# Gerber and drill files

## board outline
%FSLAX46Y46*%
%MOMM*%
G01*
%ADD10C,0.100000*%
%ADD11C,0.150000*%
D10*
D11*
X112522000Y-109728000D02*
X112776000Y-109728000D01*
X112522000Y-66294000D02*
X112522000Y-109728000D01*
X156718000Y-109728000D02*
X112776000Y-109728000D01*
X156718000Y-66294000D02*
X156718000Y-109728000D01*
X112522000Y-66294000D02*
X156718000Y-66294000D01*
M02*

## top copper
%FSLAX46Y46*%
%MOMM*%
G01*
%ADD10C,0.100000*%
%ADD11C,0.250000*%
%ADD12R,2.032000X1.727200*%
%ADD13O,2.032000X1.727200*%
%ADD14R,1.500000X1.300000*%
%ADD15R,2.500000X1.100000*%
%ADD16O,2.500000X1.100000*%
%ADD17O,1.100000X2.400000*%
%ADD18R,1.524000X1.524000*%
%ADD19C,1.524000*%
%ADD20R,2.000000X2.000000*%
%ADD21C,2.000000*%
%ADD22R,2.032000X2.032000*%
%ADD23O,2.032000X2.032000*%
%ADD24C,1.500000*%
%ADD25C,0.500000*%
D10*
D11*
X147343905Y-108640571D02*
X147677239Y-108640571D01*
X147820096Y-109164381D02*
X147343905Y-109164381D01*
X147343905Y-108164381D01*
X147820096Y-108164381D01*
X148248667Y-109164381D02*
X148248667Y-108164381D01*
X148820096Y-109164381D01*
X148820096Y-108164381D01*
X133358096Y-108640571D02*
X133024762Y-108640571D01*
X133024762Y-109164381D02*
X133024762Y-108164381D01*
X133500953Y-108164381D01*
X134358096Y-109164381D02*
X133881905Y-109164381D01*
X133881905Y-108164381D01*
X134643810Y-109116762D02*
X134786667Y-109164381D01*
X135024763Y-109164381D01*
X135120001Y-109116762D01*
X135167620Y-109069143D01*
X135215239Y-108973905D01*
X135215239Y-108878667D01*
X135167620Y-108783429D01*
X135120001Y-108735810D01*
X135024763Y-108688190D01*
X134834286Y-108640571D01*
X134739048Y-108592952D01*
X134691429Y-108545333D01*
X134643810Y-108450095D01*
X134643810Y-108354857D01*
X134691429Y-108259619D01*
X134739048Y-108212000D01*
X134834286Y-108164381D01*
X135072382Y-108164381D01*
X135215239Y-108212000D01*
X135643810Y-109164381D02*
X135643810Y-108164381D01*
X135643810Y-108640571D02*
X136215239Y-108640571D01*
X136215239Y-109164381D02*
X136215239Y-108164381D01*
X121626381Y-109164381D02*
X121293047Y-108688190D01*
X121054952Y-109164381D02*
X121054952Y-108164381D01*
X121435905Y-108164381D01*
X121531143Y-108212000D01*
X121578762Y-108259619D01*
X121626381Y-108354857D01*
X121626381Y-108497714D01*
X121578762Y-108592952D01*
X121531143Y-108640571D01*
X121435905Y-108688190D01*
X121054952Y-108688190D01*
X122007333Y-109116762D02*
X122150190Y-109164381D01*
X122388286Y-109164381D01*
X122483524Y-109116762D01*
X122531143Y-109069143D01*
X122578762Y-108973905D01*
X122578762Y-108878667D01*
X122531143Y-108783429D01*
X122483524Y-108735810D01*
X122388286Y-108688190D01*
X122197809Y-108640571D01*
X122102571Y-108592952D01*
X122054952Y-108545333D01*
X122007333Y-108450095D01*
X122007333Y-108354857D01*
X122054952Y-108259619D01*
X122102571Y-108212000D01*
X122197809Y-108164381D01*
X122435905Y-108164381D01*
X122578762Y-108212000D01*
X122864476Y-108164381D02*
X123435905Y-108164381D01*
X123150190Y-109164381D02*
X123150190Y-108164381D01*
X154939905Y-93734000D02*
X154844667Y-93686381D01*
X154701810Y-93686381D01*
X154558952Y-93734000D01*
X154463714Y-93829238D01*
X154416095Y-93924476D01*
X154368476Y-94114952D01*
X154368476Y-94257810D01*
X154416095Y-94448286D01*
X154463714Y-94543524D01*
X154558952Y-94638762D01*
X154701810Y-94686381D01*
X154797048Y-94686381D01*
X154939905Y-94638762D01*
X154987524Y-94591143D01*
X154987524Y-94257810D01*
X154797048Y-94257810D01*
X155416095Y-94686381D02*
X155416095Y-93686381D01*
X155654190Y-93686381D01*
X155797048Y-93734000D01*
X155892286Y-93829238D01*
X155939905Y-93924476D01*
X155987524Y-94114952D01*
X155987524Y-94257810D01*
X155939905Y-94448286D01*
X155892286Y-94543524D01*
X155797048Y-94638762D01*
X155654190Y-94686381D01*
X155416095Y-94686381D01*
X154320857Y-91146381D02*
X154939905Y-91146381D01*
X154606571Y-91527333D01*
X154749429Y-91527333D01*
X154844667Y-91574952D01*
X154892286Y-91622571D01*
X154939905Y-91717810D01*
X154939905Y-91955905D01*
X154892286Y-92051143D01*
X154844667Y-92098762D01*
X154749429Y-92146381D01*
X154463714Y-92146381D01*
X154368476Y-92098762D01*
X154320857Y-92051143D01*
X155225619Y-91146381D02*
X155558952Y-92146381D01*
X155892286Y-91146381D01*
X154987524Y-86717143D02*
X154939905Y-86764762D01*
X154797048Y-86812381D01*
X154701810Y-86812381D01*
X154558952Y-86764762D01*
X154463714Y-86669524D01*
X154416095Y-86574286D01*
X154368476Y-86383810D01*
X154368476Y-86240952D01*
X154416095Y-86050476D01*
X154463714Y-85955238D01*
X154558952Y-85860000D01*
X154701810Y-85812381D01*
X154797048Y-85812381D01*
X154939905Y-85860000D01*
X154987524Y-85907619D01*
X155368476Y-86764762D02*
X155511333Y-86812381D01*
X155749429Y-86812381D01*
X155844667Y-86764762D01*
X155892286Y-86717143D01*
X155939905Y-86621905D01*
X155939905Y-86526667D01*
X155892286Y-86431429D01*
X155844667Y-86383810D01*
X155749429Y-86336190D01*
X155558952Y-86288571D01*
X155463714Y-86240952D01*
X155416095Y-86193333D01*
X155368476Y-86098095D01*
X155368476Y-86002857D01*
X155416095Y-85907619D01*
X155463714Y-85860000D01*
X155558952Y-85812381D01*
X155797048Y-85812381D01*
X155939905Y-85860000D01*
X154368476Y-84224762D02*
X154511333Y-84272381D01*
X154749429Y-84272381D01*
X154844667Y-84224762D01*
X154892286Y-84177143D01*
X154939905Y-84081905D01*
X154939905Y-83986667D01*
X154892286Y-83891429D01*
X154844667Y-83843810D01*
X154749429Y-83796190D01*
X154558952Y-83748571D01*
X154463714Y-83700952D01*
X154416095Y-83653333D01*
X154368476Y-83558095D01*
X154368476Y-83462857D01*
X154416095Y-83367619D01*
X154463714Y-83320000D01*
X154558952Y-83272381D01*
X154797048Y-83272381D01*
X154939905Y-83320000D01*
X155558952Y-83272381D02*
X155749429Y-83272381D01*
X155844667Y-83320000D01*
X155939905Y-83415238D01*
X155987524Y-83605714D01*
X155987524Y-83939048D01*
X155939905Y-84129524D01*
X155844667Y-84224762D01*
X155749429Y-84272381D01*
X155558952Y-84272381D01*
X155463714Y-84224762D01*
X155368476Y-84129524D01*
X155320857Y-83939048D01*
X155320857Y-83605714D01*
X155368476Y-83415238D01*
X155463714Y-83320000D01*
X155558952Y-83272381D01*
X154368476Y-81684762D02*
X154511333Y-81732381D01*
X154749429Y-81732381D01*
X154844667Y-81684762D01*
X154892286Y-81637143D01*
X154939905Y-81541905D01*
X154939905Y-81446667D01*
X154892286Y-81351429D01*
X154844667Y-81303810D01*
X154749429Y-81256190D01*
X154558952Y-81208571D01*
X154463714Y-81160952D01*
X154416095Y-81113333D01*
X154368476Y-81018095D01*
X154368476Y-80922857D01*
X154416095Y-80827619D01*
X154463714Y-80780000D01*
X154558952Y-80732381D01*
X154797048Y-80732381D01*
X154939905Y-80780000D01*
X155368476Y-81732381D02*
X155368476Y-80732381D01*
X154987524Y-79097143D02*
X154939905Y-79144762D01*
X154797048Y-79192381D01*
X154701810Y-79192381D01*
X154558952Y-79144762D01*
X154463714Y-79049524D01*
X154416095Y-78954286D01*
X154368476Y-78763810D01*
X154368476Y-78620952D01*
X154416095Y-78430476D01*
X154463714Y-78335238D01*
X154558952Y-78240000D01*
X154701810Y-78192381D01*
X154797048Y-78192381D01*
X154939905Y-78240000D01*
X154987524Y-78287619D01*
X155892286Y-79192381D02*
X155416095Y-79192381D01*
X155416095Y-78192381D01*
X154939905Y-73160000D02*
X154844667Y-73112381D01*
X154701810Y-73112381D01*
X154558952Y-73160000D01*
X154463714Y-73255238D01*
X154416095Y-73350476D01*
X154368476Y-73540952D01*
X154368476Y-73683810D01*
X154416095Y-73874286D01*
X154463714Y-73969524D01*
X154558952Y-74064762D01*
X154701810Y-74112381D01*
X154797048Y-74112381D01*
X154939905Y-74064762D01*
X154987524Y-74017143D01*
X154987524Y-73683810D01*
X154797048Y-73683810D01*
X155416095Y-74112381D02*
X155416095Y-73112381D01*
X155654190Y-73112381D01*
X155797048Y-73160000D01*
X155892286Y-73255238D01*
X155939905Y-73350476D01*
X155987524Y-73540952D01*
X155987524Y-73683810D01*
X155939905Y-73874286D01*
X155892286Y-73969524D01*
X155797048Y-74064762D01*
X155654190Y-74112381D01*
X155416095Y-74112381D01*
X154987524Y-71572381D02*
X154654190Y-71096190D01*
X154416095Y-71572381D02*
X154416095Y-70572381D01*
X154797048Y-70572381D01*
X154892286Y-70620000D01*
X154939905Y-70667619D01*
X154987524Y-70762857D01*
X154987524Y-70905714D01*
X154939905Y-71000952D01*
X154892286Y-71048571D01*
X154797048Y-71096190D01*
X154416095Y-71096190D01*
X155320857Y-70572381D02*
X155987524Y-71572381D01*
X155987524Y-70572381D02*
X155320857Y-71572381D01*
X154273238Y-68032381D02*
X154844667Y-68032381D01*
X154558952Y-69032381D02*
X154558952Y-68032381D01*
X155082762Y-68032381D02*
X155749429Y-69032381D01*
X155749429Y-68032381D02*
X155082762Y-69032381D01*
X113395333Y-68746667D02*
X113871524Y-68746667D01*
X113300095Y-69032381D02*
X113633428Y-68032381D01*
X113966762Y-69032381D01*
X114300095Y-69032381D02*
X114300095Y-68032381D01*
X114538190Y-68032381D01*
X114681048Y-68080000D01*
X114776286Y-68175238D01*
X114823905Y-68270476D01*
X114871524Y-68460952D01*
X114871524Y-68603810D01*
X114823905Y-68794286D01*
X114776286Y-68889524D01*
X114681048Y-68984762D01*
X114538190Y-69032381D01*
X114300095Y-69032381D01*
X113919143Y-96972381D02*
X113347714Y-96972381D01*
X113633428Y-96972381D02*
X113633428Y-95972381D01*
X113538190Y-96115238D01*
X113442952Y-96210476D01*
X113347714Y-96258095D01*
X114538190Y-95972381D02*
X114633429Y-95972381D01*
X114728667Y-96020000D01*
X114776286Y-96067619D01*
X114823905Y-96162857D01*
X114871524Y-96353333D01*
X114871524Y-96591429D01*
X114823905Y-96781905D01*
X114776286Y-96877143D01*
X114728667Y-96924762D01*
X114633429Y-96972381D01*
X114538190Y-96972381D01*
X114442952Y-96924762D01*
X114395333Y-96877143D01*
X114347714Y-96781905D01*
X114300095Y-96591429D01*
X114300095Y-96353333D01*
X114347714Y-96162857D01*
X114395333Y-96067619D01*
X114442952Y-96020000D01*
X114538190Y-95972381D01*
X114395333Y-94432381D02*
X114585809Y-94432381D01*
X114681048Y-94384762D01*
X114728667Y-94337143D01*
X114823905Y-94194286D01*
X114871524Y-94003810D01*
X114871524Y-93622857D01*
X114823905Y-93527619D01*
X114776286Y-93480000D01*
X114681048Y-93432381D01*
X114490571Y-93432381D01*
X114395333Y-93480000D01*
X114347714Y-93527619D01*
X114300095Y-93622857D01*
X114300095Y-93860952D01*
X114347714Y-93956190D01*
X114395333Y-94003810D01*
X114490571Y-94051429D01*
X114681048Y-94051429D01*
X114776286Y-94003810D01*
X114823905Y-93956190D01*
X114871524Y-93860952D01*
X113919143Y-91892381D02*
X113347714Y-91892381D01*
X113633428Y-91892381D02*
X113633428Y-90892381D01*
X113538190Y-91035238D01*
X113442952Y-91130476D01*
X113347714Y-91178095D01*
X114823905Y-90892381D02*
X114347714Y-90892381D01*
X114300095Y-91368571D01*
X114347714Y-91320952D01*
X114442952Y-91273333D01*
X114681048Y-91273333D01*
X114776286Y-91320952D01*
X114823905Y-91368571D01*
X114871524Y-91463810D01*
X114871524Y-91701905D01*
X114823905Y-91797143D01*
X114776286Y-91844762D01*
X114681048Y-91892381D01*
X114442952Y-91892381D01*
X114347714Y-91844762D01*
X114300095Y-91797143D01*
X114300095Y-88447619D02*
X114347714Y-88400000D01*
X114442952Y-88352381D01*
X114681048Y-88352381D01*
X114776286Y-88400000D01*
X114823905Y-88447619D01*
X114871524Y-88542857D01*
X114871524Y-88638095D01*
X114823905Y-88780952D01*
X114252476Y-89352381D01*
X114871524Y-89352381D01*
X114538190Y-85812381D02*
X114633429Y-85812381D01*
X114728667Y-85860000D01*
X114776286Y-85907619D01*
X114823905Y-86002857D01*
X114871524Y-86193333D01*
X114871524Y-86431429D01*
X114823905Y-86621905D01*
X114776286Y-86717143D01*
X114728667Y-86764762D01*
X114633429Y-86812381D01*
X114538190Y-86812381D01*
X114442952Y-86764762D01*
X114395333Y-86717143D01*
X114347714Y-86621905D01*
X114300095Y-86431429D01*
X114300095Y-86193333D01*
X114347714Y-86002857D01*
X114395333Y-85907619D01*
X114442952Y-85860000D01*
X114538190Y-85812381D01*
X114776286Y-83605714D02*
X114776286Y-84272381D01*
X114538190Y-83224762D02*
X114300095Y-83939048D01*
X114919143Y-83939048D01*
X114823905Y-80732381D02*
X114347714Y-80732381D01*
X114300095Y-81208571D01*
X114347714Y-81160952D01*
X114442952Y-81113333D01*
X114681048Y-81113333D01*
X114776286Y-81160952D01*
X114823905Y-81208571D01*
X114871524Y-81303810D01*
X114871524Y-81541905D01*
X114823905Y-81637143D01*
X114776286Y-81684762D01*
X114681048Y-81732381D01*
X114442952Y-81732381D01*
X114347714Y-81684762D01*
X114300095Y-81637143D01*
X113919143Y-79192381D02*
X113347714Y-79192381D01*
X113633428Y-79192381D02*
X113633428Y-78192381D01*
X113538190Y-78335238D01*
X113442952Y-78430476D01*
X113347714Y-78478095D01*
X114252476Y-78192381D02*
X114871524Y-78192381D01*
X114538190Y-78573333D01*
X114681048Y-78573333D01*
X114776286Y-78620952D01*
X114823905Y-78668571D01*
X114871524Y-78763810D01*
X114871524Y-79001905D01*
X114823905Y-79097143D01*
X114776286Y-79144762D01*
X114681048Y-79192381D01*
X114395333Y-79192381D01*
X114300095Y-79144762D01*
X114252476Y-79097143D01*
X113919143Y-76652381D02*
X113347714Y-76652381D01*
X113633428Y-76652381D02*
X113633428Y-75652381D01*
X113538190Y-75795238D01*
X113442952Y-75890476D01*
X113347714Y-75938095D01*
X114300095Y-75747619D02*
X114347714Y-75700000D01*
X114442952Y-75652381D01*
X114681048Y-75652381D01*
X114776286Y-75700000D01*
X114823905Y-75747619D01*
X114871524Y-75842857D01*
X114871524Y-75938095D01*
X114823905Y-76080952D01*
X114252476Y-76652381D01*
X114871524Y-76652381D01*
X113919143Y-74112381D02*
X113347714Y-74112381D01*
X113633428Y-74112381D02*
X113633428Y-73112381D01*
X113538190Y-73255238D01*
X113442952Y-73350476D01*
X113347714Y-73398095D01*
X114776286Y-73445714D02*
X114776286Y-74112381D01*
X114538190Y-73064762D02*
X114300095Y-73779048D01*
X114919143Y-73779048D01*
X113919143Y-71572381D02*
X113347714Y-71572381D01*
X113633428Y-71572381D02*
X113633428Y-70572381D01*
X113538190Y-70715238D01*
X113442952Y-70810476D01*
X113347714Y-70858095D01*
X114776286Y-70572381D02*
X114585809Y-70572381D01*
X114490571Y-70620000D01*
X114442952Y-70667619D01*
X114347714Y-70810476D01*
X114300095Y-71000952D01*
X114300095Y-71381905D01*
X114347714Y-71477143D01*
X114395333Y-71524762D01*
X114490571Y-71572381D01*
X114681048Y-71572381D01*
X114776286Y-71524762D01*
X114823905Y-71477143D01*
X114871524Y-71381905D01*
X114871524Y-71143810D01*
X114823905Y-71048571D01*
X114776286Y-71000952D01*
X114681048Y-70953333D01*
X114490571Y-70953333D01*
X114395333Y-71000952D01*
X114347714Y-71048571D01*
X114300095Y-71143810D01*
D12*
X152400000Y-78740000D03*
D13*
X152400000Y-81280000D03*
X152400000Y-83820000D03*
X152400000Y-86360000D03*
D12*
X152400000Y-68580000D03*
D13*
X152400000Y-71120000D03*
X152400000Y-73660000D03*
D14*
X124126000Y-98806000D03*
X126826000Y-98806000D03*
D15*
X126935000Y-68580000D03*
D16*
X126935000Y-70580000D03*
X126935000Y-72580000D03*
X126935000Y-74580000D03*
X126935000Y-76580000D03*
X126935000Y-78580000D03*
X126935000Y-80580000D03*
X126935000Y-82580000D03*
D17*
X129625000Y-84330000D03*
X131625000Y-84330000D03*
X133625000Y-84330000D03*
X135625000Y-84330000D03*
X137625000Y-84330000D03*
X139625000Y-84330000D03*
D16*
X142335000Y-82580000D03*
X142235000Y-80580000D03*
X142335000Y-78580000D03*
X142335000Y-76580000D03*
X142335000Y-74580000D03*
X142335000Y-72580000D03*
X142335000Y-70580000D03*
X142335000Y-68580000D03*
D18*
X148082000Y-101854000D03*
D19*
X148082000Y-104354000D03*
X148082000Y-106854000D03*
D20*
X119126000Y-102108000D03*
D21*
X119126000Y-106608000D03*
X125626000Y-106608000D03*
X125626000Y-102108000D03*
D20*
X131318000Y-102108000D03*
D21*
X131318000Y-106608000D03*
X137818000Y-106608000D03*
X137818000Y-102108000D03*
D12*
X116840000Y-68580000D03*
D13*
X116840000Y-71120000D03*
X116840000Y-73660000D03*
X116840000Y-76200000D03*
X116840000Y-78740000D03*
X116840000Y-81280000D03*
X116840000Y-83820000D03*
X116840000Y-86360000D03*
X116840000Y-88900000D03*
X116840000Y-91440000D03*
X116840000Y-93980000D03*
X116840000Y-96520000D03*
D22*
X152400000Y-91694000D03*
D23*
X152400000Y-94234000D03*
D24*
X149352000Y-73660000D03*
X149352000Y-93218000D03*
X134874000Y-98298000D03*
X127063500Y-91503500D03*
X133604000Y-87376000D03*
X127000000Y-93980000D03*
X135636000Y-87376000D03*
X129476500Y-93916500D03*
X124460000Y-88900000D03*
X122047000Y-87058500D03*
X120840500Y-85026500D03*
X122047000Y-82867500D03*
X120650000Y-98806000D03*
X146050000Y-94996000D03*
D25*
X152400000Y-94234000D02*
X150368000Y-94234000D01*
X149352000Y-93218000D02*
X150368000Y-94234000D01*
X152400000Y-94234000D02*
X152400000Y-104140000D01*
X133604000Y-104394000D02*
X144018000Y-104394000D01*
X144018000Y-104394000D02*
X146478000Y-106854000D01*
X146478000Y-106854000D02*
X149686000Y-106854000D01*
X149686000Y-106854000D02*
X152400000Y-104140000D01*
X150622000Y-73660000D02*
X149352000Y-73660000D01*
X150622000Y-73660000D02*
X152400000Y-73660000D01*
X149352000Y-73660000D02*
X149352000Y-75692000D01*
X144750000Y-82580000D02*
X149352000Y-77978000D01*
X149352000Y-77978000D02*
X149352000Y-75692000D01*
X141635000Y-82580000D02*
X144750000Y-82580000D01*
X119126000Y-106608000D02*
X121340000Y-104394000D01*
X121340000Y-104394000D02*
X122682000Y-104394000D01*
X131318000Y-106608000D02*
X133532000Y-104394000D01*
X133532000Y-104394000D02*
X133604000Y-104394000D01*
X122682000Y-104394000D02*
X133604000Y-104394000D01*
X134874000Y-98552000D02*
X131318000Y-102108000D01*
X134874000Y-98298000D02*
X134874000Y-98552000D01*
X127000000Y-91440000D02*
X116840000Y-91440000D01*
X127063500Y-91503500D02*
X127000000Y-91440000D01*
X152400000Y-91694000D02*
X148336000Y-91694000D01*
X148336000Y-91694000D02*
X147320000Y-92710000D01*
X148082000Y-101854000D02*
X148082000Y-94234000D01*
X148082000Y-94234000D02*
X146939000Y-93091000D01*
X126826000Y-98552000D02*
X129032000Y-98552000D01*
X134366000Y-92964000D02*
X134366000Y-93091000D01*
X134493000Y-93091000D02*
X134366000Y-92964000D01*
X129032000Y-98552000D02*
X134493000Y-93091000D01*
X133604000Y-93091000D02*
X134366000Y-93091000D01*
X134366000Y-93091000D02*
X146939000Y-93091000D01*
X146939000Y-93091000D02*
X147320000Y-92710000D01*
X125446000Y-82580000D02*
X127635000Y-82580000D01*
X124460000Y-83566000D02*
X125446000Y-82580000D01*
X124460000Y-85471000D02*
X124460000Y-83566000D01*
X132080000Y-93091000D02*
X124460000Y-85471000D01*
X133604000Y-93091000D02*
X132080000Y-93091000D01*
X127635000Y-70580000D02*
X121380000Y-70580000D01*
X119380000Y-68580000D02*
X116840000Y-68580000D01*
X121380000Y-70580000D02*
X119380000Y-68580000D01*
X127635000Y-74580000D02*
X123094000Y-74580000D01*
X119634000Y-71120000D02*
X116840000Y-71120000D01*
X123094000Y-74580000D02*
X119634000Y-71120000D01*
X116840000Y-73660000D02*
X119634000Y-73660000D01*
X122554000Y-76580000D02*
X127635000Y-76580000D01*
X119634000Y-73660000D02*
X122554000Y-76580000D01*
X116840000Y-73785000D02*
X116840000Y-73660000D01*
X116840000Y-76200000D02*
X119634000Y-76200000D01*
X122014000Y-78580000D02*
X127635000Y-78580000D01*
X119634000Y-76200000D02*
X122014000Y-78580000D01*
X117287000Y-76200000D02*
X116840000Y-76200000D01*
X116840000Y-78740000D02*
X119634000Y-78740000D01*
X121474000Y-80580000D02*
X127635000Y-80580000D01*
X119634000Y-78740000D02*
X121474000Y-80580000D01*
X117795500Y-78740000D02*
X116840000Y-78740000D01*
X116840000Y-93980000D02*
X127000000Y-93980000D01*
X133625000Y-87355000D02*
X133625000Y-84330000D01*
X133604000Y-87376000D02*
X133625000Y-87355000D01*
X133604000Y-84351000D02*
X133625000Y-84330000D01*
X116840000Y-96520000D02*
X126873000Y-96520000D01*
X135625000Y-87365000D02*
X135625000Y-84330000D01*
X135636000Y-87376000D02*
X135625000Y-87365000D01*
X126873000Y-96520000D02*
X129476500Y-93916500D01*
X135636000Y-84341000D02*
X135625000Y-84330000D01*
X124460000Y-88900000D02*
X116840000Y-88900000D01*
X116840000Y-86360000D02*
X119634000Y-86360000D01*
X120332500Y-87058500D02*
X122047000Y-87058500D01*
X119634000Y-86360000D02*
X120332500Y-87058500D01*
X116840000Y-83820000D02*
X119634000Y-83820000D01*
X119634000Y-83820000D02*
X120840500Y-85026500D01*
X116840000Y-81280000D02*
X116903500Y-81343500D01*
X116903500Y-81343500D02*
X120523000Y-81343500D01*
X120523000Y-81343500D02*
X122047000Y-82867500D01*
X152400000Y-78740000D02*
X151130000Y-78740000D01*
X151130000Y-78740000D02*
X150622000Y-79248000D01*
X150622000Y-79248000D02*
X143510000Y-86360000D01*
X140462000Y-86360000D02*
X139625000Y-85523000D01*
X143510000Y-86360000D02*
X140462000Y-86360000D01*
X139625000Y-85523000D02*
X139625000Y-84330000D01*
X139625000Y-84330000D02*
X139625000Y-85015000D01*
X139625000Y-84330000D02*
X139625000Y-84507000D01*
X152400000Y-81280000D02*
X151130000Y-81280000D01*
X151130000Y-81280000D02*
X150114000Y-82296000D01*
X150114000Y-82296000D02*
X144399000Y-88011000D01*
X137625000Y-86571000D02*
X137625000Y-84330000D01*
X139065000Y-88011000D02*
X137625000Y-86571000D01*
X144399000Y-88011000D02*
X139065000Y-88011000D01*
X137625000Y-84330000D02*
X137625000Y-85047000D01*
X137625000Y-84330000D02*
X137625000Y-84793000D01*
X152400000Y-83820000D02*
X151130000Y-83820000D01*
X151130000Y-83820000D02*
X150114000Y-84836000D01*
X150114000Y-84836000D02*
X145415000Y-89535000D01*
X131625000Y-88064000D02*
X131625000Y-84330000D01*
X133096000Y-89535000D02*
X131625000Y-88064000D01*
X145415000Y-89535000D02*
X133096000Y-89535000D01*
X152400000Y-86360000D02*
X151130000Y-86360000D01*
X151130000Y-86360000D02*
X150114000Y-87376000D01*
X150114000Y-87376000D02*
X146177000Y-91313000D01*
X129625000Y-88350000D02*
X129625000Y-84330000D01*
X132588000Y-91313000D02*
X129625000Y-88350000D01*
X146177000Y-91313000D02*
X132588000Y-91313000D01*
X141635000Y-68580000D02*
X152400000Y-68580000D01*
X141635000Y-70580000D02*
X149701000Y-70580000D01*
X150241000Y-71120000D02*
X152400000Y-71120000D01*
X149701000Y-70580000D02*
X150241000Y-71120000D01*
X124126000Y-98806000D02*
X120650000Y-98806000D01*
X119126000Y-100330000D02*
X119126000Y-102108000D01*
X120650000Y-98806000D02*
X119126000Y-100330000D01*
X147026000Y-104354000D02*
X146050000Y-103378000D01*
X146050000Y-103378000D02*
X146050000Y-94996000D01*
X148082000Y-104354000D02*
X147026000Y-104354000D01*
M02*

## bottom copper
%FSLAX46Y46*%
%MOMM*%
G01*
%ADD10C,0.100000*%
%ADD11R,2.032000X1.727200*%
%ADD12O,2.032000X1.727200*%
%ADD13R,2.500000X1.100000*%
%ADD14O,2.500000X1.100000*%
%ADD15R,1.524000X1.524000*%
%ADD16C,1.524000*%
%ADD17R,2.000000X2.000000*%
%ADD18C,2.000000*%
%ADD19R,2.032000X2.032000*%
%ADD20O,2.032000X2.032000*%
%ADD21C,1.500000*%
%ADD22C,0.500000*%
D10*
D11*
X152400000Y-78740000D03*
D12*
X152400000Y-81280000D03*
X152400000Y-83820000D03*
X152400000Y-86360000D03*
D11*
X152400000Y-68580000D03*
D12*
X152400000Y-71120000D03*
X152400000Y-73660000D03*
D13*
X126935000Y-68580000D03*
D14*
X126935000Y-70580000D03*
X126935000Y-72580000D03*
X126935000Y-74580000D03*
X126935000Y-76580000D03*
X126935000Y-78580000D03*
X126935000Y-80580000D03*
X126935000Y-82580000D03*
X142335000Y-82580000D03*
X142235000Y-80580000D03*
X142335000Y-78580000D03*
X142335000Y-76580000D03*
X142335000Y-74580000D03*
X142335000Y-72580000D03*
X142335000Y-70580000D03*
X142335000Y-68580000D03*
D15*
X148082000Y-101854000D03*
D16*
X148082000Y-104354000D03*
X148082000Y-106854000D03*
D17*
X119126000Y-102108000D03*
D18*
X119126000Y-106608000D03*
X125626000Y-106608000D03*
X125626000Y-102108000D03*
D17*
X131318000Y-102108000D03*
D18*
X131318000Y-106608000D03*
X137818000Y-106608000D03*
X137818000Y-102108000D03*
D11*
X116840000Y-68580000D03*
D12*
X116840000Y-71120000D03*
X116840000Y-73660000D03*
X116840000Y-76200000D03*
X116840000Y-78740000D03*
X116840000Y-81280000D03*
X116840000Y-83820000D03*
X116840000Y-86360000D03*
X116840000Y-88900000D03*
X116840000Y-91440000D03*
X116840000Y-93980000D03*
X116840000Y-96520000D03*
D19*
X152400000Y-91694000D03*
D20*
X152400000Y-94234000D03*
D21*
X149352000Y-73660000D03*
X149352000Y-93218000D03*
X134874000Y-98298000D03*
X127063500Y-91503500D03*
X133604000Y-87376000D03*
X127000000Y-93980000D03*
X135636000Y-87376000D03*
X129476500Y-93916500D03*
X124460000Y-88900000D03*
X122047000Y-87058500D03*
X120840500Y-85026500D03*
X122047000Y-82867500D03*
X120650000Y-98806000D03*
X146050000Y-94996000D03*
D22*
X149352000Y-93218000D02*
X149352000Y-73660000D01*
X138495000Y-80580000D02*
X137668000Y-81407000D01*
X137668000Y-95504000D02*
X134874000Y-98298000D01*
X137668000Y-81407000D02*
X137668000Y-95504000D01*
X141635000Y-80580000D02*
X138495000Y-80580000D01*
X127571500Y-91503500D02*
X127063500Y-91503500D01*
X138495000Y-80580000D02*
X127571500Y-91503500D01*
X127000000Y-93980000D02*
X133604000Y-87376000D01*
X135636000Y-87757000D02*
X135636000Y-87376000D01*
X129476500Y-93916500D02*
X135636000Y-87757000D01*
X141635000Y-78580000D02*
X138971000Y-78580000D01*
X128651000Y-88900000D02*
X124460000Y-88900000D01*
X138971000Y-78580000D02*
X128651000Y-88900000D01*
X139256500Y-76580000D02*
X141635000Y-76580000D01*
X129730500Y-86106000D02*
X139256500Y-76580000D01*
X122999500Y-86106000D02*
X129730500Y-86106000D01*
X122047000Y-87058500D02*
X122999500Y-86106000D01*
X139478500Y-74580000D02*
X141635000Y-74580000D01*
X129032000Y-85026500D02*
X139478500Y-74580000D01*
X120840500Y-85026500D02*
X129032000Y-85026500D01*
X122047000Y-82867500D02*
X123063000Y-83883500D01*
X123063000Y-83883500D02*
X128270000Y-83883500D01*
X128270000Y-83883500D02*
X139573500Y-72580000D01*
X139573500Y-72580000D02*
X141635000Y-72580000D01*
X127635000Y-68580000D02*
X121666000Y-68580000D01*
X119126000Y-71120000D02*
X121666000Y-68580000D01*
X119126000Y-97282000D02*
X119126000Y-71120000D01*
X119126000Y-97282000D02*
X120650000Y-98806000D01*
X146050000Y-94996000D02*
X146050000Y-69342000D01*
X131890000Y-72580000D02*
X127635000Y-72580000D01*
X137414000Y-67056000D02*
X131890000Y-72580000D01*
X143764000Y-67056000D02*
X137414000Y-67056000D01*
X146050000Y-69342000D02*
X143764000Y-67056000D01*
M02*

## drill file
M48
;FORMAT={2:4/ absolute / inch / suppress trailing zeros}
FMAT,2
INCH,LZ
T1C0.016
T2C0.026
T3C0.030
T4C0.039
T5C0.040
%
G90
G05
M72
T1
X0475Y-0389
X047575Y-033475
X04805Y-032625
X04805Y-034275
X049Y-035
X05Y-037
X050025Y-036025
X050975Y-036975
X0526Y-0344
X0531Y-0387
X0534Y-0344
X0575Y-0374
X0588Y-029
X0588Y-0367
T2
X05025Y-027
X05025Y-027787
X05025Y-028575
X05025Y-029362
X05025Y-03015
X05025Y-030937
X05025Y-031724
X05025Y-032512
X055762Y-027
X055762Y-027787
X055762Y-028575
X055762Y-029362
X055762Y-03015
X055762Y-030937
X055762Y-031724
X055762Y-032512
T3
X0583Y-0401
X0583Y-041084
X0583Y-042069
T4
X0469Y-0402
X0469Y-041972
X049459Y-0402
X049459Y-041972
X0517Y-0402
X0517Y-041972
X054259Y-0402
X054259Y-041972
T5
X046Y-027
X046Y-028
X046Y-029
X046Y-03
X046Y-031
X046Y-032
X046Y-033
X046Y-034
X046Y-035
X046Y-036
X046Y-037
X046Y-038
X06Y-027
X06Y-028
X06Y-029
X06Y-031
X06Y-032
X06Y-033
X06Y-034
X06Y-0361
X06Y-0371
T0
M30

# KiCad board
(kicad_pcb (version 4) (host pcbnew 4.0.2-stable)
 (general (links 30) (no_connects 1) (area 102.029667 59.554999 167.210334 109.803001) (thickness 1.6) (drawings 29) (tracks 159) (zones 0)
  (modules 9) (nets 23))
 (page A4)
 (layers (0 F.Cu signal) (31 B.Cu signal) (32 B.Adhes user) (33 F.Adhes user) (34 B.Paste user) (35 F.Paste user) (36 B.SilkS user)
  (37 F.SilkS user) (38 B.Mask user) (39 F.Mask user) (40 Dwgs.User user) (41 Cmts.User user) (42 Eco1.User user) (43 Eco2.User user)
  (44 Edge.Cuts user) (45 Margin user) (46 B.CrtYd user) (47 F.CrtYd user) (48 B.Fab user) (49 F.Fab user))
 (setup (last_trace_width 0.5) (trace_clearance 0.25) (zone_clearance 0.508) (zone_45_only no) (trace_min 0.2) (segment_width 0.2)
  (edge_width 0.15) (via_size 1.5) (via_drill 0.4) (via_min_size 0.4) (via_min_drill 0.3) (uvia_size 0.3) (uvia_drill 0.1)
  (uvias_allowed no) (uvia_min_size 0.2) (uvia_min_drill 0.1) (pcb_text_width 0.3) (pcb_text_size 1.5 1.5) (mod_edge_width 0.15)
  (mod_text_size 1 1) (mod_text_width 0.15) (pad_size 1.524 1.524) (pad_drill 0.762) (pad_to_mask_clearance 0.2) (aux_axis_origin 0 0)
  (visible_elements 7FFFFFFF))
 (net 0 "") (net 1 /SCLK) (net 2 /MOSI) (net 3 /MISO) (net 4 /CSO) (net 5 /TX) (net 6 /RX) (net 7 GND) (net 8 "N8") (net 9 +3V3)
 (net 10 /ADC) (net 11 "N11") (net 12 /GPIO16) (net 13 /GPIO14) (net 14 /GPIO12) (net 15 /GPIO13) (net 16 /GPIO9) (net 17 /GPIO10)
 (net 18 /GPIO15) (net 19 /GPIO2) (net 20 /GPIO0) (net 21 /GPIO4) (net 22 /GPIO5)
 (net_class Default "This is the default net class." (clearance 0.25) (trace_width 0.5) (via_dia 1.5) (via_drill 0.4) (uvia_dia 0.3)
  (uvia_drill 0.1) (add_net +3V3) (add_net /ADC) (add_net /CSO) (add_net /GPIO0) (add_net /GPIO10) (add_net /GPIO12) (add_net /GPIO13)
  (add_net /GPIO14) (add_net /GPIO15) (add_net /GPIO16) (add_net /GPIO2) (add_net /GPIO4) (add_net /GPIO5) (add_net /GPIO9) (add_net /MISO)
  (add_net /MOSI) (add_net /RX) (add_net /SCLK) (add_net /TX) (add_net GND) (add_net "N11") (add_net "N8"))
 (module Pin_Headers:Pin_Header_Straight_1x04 (layer F.Cu) (at 152.4 78.74)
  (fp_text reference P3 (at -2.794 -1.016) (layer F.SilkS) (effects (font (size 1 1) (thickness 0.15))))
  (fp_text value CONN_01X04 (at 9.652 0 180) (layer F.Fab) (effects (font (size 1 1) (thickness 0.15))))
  (pad 1 thru_hole rect (at 0 0) (size 2.032 1.7272) (drill 1.016) (layers *.Cu *.Mask F.SilkS) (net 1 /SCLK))
  (pad 2 thru_hole oval (at 0 2.54) (size 2.032 1.7272) (drill 1.016) (layers *.Cu *.Mask F.SilkS) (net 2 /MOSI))
  (pad 3 thru_hole oval (at 0 5.08) (size 2.032 1.7272) (drill 1.016) (layers *.Cu *.Mask F.SilkS) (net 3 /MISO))
  (pad 4 thru_hole oval (at 0 7.62) (size 2.032 1.7272) (drill 1.016) (layers *.Cu *.Mask F.SilkS) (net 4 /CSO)))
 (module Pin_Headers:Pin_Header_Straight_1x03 (layer F.Cu) (at 152.4 68.58)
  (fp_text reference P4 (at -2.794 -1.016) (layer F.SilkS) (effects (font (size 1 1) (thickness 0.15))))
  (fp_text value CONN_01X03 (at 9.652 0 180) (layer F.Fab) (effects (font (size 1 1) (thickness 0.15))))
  (pad 1 thru_hole rect (at 0 0) (size 2.032 1.7272) (drill 1.016) (layers *.Cu *.Mask F.SilkS) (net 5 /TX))
  (pad 2 thru_hole oval (at 0 2.54) (size 2.032 1.7272) (drill 1.016) (layers *.Cu *.Mask F.SilkS) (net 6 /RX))
  (pad 3 thru_hole oval (at 0 5.08) (size 2.032 1.7272) (drill 1.016) (layers *.Cu *.Mask F.SilkS) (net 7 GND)))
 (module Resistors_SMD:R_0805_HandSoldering (layer F.Cu) (at 125.476 98.806)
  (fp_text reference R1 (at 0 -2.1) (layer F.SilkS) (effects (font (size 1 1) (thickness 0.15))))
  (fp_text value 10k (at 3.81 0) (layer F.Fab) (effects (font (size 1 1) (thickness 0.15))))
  (pad 1 smd rect (at -1.35 0) (size 1.5 1.3) (layers F.Cu F.Paste F.Mask) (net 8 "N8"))
  (pad 2 smd rect (at 1.35 0) (size 1.5 1.3) (layers F.Cu F.Paste F.Mask) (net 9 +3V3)))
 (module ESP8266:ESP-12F (layer F.Cu) (at 127.635 68.58)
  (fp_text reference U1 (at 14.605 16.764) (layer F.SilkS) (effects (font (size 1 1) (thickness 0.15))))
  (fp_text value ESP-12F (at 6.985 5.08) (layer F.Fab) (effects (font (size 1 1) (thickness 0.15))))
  (pad 1 thru_hole rect (at 0 0) (size 2.5 1.1) (drill 0.65 (offset -0.7 0)) (layers *.Cu *.Mask F.SilkS) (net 8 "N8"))
  (pad 2 thru_hole oval (at 0 2) (size 2.5 1.1) (drill 0.65 (offset -0.7 0)) (layers *.Cu *.Mask F.SilkS) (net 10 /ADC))
  (pad 3 thru_hole oval (at 0 4) (size 2.5 1.1) (drill 0.65 (offset -0.7 0)) (layers *.Cu *.Mask F.SilkS) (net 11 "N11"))
  (pad 4 thru_hole oval (at 0 6) (size 2.5 1.1) (drill 0.65 (offset -0.7 0)) (layers *.Cu *.Mask F.SilkS) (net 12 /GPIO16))
  (pad 5 thru_hole oval (at 0 8) (size 2.5 1.1) (drill 0.65 (offset -0.7 0)) (layers *.Cu *.Mask F.SilkS) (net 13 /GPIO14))
  (pad 6 thru_hole oval (at 0 10) (size 2.5 1.1) (drill 0.65 (offset -0.7 0)) (layers *.Cu *.Mask F.SilkS) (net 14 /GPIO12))
  (pad 7 thru_hole oval (at 0 12) (size 2.5 1.1) (drill 0.65 (offset -0.7 0)) (layers *.Cu *.Mask F.SilkS) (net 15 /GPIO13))
  (pad 8 thru_hole oval (at 0 14) (size 2.5 1.1) (drill 0.65 (offset -0.7 0)) (layers *.Cu *.Mask F.SilkS) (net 9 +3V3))
  (pad 9 smd oval (at 1.99 15.75 90) (size 2.4 1.1) (layers F.Cu F.Paste F.Mask) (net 4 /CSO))
  (pad 10 smd oval (at 3.99 15.75 90) (size 2.4 1.1) (layers F.Cu F.Paste F.Mask) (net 3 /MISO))
  (pad 11 smd oval (at 5.99 15.75 90) (size 2.4 1.1) (layers F.Cu F.Paste F.Mask) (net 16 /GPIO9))
  (pad 12 smd oval (at 7.99 15.75 90) (size 2.4 1.1) (layers F.Cu F.Paste F.Mask) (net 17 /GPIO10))
  (pad 13 smd oval (at 9.99 15.75 90) (size 2.4 1.1) (layers F.Cu F.Paste F.Mask) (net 2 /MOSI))
  (pad 14 smd oval (at 11.99 15.75 90) (size 2.4 1.1) (layers F.Cu F.Paste F.Mask) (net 1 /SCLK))
  (pad 15 thru_hole oval (at 14 14) (size 2.5 1.1) (drill 0.65 (offset 0.7 0)) (layers *.Cu *.Mask F.SilkS) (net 7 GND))
  (pad 16 thru_hole oval (at 14 12) (size 2.5 1.1) (drill 0.65 (offset 0.6 0)) (layers *.Cu *.Mask F.SilkS) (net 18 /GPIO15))
  (pad 17 thru_hole oval (at 14 10) (size 2.5 1.1) (drill 0.65 (offset 0.7 0)) (layers *.Cu *.Mask F.SilkS) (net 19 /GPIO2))
  (pad 18 thru_hole oval (at 14 8) (size 2.5 1.1) (drill 0.65 (offset 0.7 0)) (layers *.Cu *.Mask F.SilkS) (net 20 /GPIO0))
  (pad 19 thru_hole oval (at 14 6) (size 2.5 1.1) (drill 0.65 (offset 0.7 0)) (layers *.Cu *.Mask F.SilkS) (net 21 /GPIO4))
  (pad 20 thru_hole oval (at 14 4) (size 2.5 1.1) (drill 0.65 (offset 0.7 0)) (layers *.Cu *.Mask F.SilkS) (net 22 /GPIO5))
  (pad 21 thru_hole oval (at 14 2) (size 2.5 1.1) (drill 0.65 (offset 0.7 0)) (layers *.Cu *.Mask F.SilkS) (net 6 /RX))
  (pad 22 thru_hole oval (at 14 0) (size 2.5 1.1) (drill 0.65 (offset 0.7 0)) (layers *.Cu *.Mask F.SilkS) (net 5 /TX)))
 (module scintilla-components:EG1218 (layer F.Cu) (at 148.082 101.854 270)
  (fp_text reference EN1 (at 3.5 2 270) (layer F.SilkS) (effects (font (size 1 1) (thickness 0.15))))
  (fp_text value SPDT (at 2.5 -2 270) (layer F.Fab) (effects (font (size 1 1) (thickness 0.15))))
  (pad 1 thru_hole rect (at 0 0 270) (size 1.524 1.524) (drill 0.762) (layers *.Cu *.Mask F.SilkS) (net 9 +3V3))
  (pad 2 thru_hole circle (at 2.5 0 270) (size 1.524 1.524) (drill 0.762) (layers *.Cu *.Mask F.SilkS) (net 11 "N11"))
  (pad 3 thru_hole circle (at 5 0 270) (size 1.524 1.524) (drill 0.762) (layers *.Cu *.Mask F.SilkS) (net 7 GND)))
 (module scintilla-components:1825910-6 (layer F.Cu) (at 119.126 102.108)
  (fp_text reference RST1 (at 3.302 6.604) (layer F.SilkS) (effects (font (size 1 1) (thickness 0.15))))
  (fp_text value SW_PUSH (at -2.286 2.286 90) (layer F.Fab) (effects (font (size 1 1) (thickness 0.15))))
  (pad 1 thru_hole rect (at 0 0) (size 2 2) (drill 1) (layers *.Cu *.Mask F.SilkS) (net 8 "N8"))
  (pad 2 thru_hole circle (at 0 4.5) (size 2 2) (drill 1) (layers *.Cu *.Mask F.SilkS) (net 7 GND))
  (pad 3 thru_hole circle (at 6.5 4.5) (size 2 2) (drill 1) (layers *.Cu *.Mask F.SilkS))
  (pad 4 thru_hole circle (at 6.5 0) (size 2 2) (drill 1) (layers *.Cu *.Mask F.SilkS)))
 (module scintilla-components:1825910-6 (layer F.Cu) (at 131.318 102.108)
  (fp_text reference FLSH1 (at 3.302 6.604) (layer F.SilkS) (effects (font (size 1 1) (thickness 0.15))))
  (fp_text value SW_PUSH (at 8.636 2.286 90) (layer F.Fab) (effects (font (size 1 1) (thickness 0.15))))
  (pad 1 thru_hole rect (at 0 0) (size 2 2) (drill 1) (layers *.Cu *.Mask F.SilkS) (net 18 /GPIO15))
  (pad 2 thru_hole circle (at 0 4.5) (size 2 2) (drill 1) (layers *.Cu *.Mask F.SilkS) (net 7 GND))
  (pad 3 thru_hole circle (at 6.5 4.5) (size 2 2) (drill 1) (layers *.Cu *.Mask F.SilkS))
  (pad 4 thru_hole circle (at 6.5 0) (size 2 2) (drill 1) (layers *.Cu *.Mask F.SilkS)))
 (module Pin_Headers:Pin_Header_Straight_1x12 (layer F.Cu) (at 116.84 68.58)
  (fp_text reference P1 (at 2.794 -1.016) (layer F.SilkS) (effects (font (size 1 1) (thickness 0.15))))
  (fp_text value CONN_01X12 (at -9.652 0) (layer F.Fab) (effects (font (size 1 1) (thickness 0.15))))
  (pad 1 thru_hole rect (at 0 0) (size 2.032 1.7272) (drill 1.016) (layers *.Cu *.Mask F.SilkS) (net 10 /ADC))
  (pad 2 thru_hole oval (at 0 2.54) (size 2.032 1.7272) (drill 1.016) (layers *.Cu *.Mask F.SilkS) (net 12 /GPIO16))
  (pad 3 thru_hole oval (at 0 5.08) (size 2.032 1.7272) (drill 1.016) (layers *.Cu *.Mask F.SilkS) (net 13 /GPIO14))
  (pad 4 thru_hole oval (at 0 7.62) (size 2.032 1.7272) (drill 1.016) (layers *.Cu *.Mask F.SilkS) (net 14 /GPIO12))
  (pad 5 thru_hole oval (at 0 10.16) (size 2.032 1.7272) (drill 1.016) (layers *.Cu *.Mask F.SilkS) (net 15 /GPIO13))
  (pad 6 thru_hole oval (at 0 12.7) (size 2.032 1.7272) (drill 1.016) (layers *.Cu *.Mask F.SilkS) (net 22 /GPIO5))
  (pad 7 thru_hole oval (at 0 15.24) (size 2.032 1.7272) (drill 1.016) (layers *.Cu *.Mask F.SilkS) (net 21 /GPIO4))
  (pad 8 thru_hole oval (at 0 17.78) (size 2.032 1.7272) (drill 1.016) (layers *.Cu *.Mask F.SilkS) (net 20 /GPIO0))
  (pad 9 thru_hole oval (at 0 20.32) (size 2.032 1.7272) (drill 1.016) (layers *.Cu *.Mask F.SilkS) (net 19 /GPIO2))
  (pad 10 thru_hole oval (at 0 22.86) (size 2.032 1.7272) (drill 1.016) (layers *.Cu *.Mask F.SilkS) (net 18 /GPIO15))
  (pad 11 thru_hole oval (at 0 25.4) (size 2.032 1.7272) (drill 1.016) (layers *.Cu *.Mask F.SilkS) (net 16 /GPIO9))
  (pad 12 thru_hole oval (at 0 27.94) (size 2.032 1.7272) (drill 1.016) (layers *.Cu *.Mask F.SilkS) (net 17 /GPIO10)))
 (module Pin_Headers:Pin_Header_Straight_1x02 (layer F.Cu) (at 152.4 91.694)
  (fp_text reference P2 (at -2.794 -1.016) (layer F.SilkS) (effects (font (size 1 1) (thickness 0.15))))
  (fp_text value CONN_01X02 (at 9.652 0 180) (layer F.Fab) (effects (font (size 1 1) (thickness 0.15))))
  (pad 1 thru_hole rect (at 0 0) (size 2.032 2.032) (drill 1.016) (layers *.Cu *.Mask F.SilkS) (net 9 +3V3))
  (pad 2 thru_hole oval (at 0 2.54) (size 2.032 2.032) (drill 1.016) (layers *.Cu *.Mask F.SilkS) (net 7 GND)))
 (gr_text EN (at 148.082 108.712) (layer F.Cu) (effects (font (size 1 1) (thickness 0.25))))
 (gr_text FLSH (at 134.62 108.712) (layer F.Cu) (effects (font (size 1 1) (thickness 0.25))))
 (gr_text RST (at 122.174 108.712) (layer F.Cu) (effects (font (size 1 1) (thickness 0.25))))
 (gr_line (start 112.522 109.728) (end 112.776 109.728) (angle 90) (layer Edge.Cuts) (width 0.15))
 (gr_line (start 112.522 66.294) (end 112.522 109.728) (angle 90) (layer Edge.Cuts) (width 0.15))
 (gr_line (start 156.718 109.728) (end 112.776 109.728) (angle 90) (layer Edge.Cuts) (width 0.15))
 (gr_line (start 156.718 66.294) (end 156.718 109.728) (angle 90) (layer Edge.Cuts) (width 0.15))
 (gr_line (start 112.522 66.294) (end 156.718 66.294) (angle 90) (layer Edge.Cuts) (width 0.15))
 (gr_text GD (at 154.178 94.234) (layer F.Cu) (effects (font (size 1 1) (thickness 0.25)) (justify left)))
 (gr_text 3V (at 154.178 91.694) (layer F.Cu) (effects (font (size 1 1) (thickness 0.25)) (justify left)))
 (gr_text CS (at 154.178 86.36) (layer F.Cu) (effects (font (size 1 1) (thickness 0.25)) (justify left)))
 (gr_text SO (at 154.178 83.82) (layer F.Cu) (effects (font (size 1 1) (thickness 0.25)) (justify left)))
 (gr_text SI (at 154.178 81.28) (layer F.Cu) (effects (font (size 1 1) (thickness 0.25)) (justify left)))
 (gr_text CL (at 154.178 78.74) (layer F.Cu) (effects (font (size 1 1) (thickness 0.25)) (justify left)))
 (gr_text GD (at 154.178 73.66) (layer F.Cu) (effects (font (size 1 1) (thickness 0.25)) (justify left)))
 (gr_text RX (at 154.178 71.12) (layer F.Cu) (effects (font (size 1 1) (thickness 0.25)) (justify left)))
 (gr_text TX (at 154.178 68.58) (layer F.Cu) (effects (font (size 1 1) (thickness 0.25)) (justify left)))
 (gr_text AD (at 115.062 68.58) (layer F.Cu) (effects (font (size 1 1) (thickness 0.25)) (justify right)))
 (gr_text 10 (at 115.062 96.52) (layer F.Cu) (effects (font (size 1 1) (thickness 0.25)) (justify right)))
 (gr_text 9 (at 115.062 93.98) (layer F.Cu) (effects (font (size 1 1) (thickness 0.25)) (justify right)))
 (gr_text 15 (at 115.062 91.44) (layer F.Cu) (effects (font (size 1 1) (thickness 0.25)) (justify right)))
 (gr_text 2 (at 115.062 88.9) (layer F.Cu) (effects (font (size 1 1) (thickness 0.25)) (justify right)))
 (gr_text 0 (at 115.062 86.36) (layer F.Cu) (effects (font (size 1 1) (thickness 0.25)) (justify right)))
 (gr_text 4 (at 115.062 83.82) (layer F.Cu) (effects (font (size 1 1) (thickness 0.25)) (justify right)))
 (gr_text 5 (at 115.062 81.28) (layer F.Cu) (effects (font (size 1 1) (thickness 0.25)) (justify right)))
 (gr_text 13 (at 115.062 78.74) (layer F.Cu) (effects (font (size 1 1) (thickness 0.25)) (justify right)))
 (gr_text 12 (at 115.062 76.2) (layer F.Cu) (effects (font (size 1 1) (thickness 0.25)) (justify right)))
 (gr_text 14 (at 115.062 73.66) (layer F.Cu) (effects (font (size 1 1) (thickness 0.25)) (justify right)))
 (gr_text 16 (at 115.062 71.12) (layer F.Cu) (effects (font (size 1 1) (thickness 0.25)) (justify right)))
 (via (at 149.352 73.66) (size 1.5) (drill 0.4) (layers F.Cu B.Cu) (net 7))
 (segment (start 152.4 94.234) (end 150.368 94.234) (width 0.5) (layer F.Cu) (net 7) (status 400000))
 (segment (start 149.352 93.218) (end 150.368 94.234) (width 0.5) (layer F.Cu) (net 7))
 (via (at 149.352 93.218) (size 1.5) (drill 0.4) (layers F.Cu B.Cu) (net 7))
 (segment (start 149.352 93.218) (end 149.352 73.66) (width 0.5) (layer B.Cu) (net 7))
 (segment (start 152.4 94.234) (end 152.4 104.14) (width 0.5) (layer F.Cu) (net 7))
 (segment (start 133.604 104.394) (end 144.018 104.394) (width 0.5) (layer F.Cu) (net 7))
 (segment (start 144.018 104.394) (end 146.478 106.854) (width 0.5) (layer F.Cu) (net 7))
 (segment (start 146.478 106.854) (end 149.686 106.854) (width 0.5) (layer F.Cu) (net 7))
 (segment (start 149.686 106.854) (end 152.4 104.14) (width 0.5) (layer F.Cu) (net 7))
 (segment (start 150.622 73.66) (end 149.352 73.66) (width 0.5) (layer F.Cu) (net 7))
 (segment (start 150.622 73.66) (end 152.4 73.66) (width 0.5) (layer F.Cu) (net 7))
 (segment (start 149.352 73.66) (end 149.352 75.692) (width 0.5) (layer F.Cu) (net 7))
 (segment (start 144.75 82.58) (end 149.352 77.978) (width 0.5) (layer F.Cu) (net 7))
 (segment (start 149.352 77.978) (end 149.352 75.692) (width 0.5) (layer F.Cu) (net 7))
 (segment (start 141.635 82.58) (end 144.75 82.58) (width 0.5) (layer F.Cu) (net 7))
 (segment (start 119.126 106.608) (end 121.34 104.394) (width 0.5) (layer F.Cu) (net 7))
 (segment (start 121.34 104.394) (end 122.682 104.394) (width 0.5) (layer F.Cu) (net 7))
 (segment (start 131.318 106.608) (end 133.532 104.394) (width 0.5) (layer F.Cu) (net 7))
 (segment (start 133.532 104.394) (end 133.604 104.394) (width 0.5) (layer F.Cu) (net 7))
 (segment (start 122.682 104.394) (end 133.604 104.394) (width 0.5) (layer F.Cu) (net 7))
 (segment (start 138.495 80.58) (end 137.668 81.407) (width 0.5) (layer B.Cu) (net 18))
 (segment (start 134.874 98.552) (end 131.318 102.108) (width 0.5) (layer F.Cu) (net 18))
 (segment (start 134.874 98.298) (end 134.874 98.552) (width 0.5) (layer F.Cu) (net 18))
 (via (at 134.874 98.298) (size 1.5) (drill 0.4) (layers F.Cu B.Cu) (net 18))
 (segment (start 137.668 95.504) (end 134.874 98.298) (width 0.5) (layer B.Cu) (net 18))
 (segment (start 137.668 81.407) (end 137.668 95.504) (width 0.5) (layer B.Cu) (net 18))
 (segment (start 141.635 80.58) (end 138.495 80.58) (width 0.5) (layer B.Cu) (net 18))
 (segment (start 127 91.44) (end 116.84 91.44) (width 0.5) (layer F.Cu) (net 18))
 (segment (start 127.0635 91.5035) (end 127 91.44) (width 0.5) (layer F.Cu) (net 18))
 (via (at 127.0635 91.5035) (size 1.5) (drill 0.4) (layers F.Cu B.Cu) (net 18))
 (segment (start 127.5715 91.5035) (end 127.0635 91.5035) (width 0.5) (layer B.Cu) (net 18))
 (segment (start 138.495 80.58) (end 127.5715 91.5035) (width 0.5) (layer B.Cu) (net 18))
 (segment (start 152.4 91.694) (end 148.336 91.694) (width 0.5) (layer F.Cu) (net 9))
 (segment (start 148.336 91.694) (end 147.32 92.71) (width 0.5) (layer F.Cu) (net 9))
 (segment (start 148.082 101.854) (end 148.082 94.234) (width 0.5) (layer F.Cu) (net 9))
 (segment (start 148.082 94.234) (end 146.939 93.091) (width 0.5) (layer F.Cu) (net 9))
 (segment (start 126.826 98.552) (end 129.032 98.552) (width 0.5) (layer F.Cu) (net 9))
 (segment (start 134.366 92.964) (end 134.366 93.091) (width 0.5) (layer F.Cu) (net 9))
 (segment (start 134.493 93.091) (end 134.366 92.964) (width 0.5) (layer F.Cu) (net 9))
 (segment (start 129.032 98.552) (end 134.493 93.091) (width 0.5) (layer F.Cu) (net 9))
 (segment (start 133.604 93.091) (end 134.366 93.091) (width 0.5) (layer F.Cu) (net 9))
 (segment (start 134.366 93.091) (end 146.939 93.091) (width 0.5) (layer F.Cu) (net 9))
 (segment (start 146.939 93.091) (end 147.32 92.71) (width 0.5) (layer F.Cu) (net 9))
 (segment (start 125.446 82.58) (end 127.635 82.58) (width 0.5) (layer F.Cu) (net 9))
 (segment (start 124.46 83.566) (end 125.446 82.58) (width 0.5) (layer F.Cu) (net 9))
 (segment (start 124.46 85.471) (end 124.46 83.566) (width 0.5) (layer F.Cu) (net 9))
 (segment (start 132.08 93.091) (end 124.46 85.471) (width 0.5) (layer F.Cu) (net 9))
 (segment (start 133.604 93.091) (end 132.08 93.091) (width 0.5) (layer F.Cu) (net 9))
 (segment (start 127.635 70.58) (end 121.38 70.58) (width 0.5) (layer F.Cu) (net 10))
 (segment (start 119.38 68.58) (end 116.84 68.58) (width 0.5) (layer F.Cu) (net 10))
 (segment (start 121.38 70.58) (end 119.38 68.58) (width 0.5) (layer F.Cu) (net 10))
 (segment (start 127.635 74.58) (end 123.094 74.58) (width 0.5) (layer F.Cu) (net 12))
 (segment (start 119.634 71.12) (end 116.84 71.12) (width 0.5) (layer F.Cu) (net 12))
 (segment (start 123.094 74.58) (end 119.634 71.12) (width 0.5) (layer F.Cu) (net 12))
 (segment (start 116.84 73.66) (end 119.634 73.66) (width 0.5) (layer F.Cu) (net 13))
 (segment (start 122.554 76.58) (end 127.635 76.58) (width 0.5) (layer F.Cu) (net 13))
 (segment (start 119.634 73.66) (end 122.554 76.58) (width 0.5) (layer F.Cu) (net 13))
 (segment (start 116.84 73.785) (end 116.84 73.66) (width 0.5) (layer F.Cu) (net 13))
 (segment (start 116.84 76.2) (end 119.634 76.2) (width 0.5) (layer F.Cu) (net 14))
 (segment (start 122.014 78.58) (end 127.635 78.58) (width 0.5) (layer F.Cu) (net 14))
 (segment (start 119.634 76.2) (end 122.014 78.58) (width 0.5) (layer F.Cu) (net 14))
 (segment (start 117.287 76.2) (end 116.84 76.2) (width 0.5) (layer F.Cu) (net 14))
 (segment (start 116.84 78.74) (end 119.634 78.74) (width 0.5) (layer F.Cu) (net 15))
 (segment (start 121.474 80.58) (end 127.635 80.58) (width 0.5) (layer F.Cu) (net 15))
 (segment (start 119.634 78.74) (end 121.474 80.58) (width 0.5) (layer F.Cu) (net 15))
 (segment (start 117.7955 78.74) (end 116.84 78.74) (width 0.5) (layer F.Cu) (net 15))
 (segment (start 116.84 93.98) (end 127 93.98) (width 0.5) (layer F.Cu) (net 16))
 (segment (start 133.625 87.355) (end 133.625 84.33) (width 0.5) (layer F.Cu) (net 16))
 (segment (start 133.604 87.376) (end 133.625 87.355) (width 0.5) (layer F.Cu) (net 16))
 (via (at 133.604 87.376) (size 1.5) (drill 0.4) (layers F.Cu B.Cu) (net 16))
 (segment (start 127 93.98) (end 133.604 87.376) (width 0.5) (layer B.Cu) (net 16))
 (via (at 127 93.98) (size 1.5) (drill 0.4) (layers F.Cu B.Cu) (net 16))
 (segment (start 133.604 84.351) (end 133.625 84.33) (width 0.5) (layer F.Cu) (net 16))
 (segment (start 116.84 96.52) (end 126.873 96.52) (width 0.5) (layer F.Cu) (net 17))
 (segment (start 135.625 87.365) (end 135.625 84.33) (width 0.5) (layer F.Cu) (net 17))
 (segment (start 135.636 87.376) (end 135.625 87.365) (width 0.5) (layer F.Cu) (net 17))
 (via (at 135.636 87.376) (size 1.5) (drill 0.4) (layers F.Cu B.Cu) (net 17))
 (segment (start 135.636 87.757) (end 135.636 87.376) (width 0.5) (layer B.Cu) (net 17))
 (segment (start 129.4765 93.9165) (end 135.636 87.757) (width 0.5) (layer B.Cu) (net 17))
 (via (at 129.4765 93.9165) (size 1.5) (drill 0.4) (layers F.Cu B.Cu) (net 17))
 (segment (start 126.873 96.52) (end 129.4765 93.9165) (width 0.5) (layer F.Cu) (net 17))
 (segment (start 135.636 84.341) (end 135.625 84.33) (width 0.5) (layer F.Cu) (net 17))
 (segment (start 141.635 78.58) (end 138.971 78.58) (width 0.5) (layer B.Cu) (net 19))
 (segment (start 124.46 88.9) (end 116.84 88.9) (width 0.5) (layer F.Cu) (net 19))
 (via (at 124.46 88.9) (size 1.5) (drill 0.4) (layers F.Cu B.Cu) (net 19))
 (segment (start 128.651 88.9) (end 124.46 88.9) (width 0.5) (layer B.Cu) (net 19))
 (segment (start 138.971 78.58) (end 128.651 88.9) (width 0.5) (layer B.Cu) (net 19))
 (segment (start 116.84 86.36) (end 119.634 86.36) (width 0.5) (layer F.Cu) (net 20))
 (segment (start 139.2565 76.58) (end 141.635 76.58) (width 0.5) (layer B.Cu) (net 20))
 (segment (start 129.7305 86.106) (end 139.2565 76.58) (width 0.5) (layer B.Cu) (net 20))
 (segment (start 122.9995 86.106) (end 129.7305 86.106) (width 0.5) (layer B.Cu) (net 20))
 (segment (start 122.047 87.0585) (end 122.9995 86.106) (width 0.5) (layer B.Cu) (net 20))
 (via (at 122.047 87.0585) (size 1.5) (drill 0.4) (layers F.Cu B.Cu) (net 20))
 (segment (start 120.3325 87.0585) (end 122.047 87.0585) (width 0.5) (layer F.Cu) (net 20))
 (segment (start 119.634 86.36) (end 120.3325 87.0585) (width 0.5) (layer F.Cu) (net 20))
 (segment (start 116.84 83.82) (end 119.634 83.82) (width 0.5) (layer F.Cu) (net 21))
 (segment (start 139.4785 74.58) (end 141.635 74.58) (width 0.5) (layer B.Cu) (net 21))
 (segment (start 129.032 85.0265) (end 139.4785 74.58) (width 0.5) (layer B.Cu) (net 21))
 (segment (start 120.8405 85.0265) (end 129.032 85.0265) (width 0.5) (layer B.Cu) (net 21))
 (via (at 120.8405 85.0265) (size 1.5) (drill 0.4) (layers F.Cu B.Cu) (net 21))
 (segment (start 119.634 83.82) (end 120.8405 85.0265) (width 0.5) (layer F.Cu) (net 21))
 (segment (start 116.84 81.28) (end 116.9035 81.3435) (width 0.5) (layer F.Cu) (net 22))
 (segment (start 116.9035 81.3435) (end 120.523 81.3435) (width 0.5) (layer F.Cu) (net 22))
 (segment (start 120.523 81.3435) (end 122.047 82.8675) (width 0.5) (layer F.Cu) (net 22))
 (via (at 122.047 82.8675) (size 1.5) (drill 0.4) (layers F.Cu B.Cu) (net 22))
 (segment (start 122.047 82.8675) (end 123.063 83.8835) (width 0.5) (layer B.Cu) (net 22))
 (segment (start 123.063 83.8835) (end 128.27 83.8835) (width 0.5) (layer B.Cu) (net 22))
 (segment (start 128.27 83.8835) (end 139.5735 72.58) (width 0.5) (layer B.Cu) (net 22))
 (segment (start 139.5735 72.58) (end 141.635 72.58) (width 0.5) (layer B.Cu) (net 22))
 (segment (start 152.4 78.74) (end 151.13 78.74) (width 0.5) (layer F.Cu) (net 1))
 (segment (start 151.13 78.74) (end 150.622 79.248) (width 0.5) (layer F.Cu) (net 1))
 (segment (start 150.622 79.248) (end 143.51 86.36) (width 0.5) (layer F.Cu) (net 1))
 (segment (start 140.462 86.36) (end 139.625 85.523) (width 0.5) (layer F.Cu) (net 1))
 (segment (start 143.51 86.36) (end 140.462 86.36) (width 0.5) (layer F.Cu) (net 1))
 (segment (start 139.625 85.523) (end 139.625 84.33) (width 0.5) (layer F.Cu) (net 1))
 (segment (start 139.625 84.33) (end 139.625 85.015) (width 0.5) (layer F.Cu) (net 1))
 (segment (start 139.625 84.33) (end 139.625 84.507) (width 0.5) (layer F.Cu) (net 1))
 (segment (start 152.4 81.28) (end 151.13 81.28) (width 0.5) (layer F.Cu) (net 2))
 (segment (start 151.13 81.28) (end 150.114 82.296) (width 0.5) (layer F.Cu) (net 2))
 (segment (start 150.114 82.296) (end 144.399 88.011) (width 0.5) (layer F.Cu) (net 2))
 (segment (start 137.625 86.571) (end 137.625 84.33) (width 0.5) (layer F.Cu) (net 2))
 (segment (start 139.065 88.011) (end 137.625 86.571) (width 0.5) (layer F.Cu) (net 2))
 (segment (start 144.399 88.011) (end 139.065 88.011) (width 0.5) (layer F.Cu) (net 2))
 (segment (start 137.625 84.33) (end 137.625 85.047) (width 0.5) (layer F.Cu) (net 2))
 (segment (start 137.625 84.33) (end 137.625 84.793) (width 0.5) (layer F.Cu) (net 2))
 (segment (start 152.4 83.82) (end 151.13 83.82) (width 0.5) (layer F.Cu) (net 3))
 (segment (start 151.13 83.82) (end 150.114 84.836) (width 0.5) (layer F.Cu) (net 3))
 (segment (start 150.114 84.836) (end 145.415 89.535) (width 0.5) (layer F.Cu) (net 3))
 (segment (start 131.625 88.064) (end 131.625 84.33) (width 0.5) (layer F.Cu) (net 3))
 (segment (start 133.096 89.535) (end 131.625 88.064) (width 0.5) (layer F.Cu) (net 3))
 (segment (start 145.415 89.535) (end 133.096 89.535) (width 0.5) (layer F.Cu) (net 3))
 (segment (start 152.4 86.36) (end 151.13 86.36) (width 0.5) (layer F.Cu) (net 4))
 (segment (start 151.13 86.36) (end 150.114 87.376) (width 0.5) (layer F.Cu) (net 4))
 (segment (start 150.114 87.376) (end 146.177 91.313) (width 0.5) (layer F.Cu) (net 4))
 (segment (start 129.625 88.35) (end 129.625 84.33) (width 0.5) (layer F.Cu) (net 4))
 (segment (start 132.588 91.313) (end 129.625 88.35) (width 0.5) (layer F.Cu) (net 4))
 (segment (start 146.177 91.313) (end 132.588 91.313) (width 0.5) (layer F.Cu) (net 4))
 (segment (start 141.635 68.58) (end 152.4 68.58) (width 0.5) (layer F.Cu) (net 5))
 (segment (start 141.635 70.58) (end 149.701 70.58) (width 0.5) (layer F.Cu) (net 6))
 (segment (start 150.241 71.12) (end 152.4 71.12) (width 0.5) (layer F.Cu) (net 6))
 (segment (start 149.701 70.58) (end 150.241 71.12) (width 0.5) (layer F.Cu) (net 6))
 (via (at 120.65 98.806) (size 1.5) (drill 0.4) (layers F.Cu B.Cu) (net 8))
 (segment (start 127.635 68.58) (end 121.666 68.58) (width 0.5) (layer B.Cu) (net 8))
 (segment (start 119.126 71.12) (end 121.666 68.58) (width 0.5) (layer B.Cu) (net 8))
 (segment (start 119.126 97.282) (end 119.126 71.12) (width 0.5) (layer B.Cu) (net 8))
 (segment (start 119.126 97.282) (end 120.65 98.806) (width 0.5) (layer B.Cu) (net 8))
 (segment (start 124.126 98.806) (end 120.65 98.806) (width 0.5) (layer F.Cu) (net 8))
 (segment (start 119.126 100.33) (end 119.126 102.108) (width 0.5) (layer F.Cu) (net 8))
 (segment (start 120.65 98.806) (end 119.126 100.33) (width 0.5) (layer F.Cu) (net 8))
 (segment (start 146.05 94.996) (end 146.05 69.342) (width 0.5) (layer B.Cu) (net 11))
 (segment (start 147.026 104.354) (end 146.05 103.378) (width 0.5) (layer F.Cu) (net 11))
 (segment (start 146.05 103.378) (end 146.05 94.996) (width 0.5) (layer F.Cu) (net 11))
 (via (at 146.05 94.996) (size 1.5) (drill 0.4) (layers F.Cu B.Cu) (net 11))
 (segment (start 148.082 104.354) (end 147.026 104.354) (width 0.5) (layer F.Cu) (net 11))
 (segment (start 131.89 72.58) (end 127.635 72.58) (width 0.5) (layer B.Cu) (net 11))
 (segment (start 137.414 67.056) (end 131.89 72.58) (width 0.5) (layer B.Cu) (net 11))
 (segment (start 143.764 67.056) (end 137.414 67.056) (width 0.5) (layer B.Cu) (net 11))
 (segment (start 146.05 69.342) (end 143.764 67.056) (width 0.5) (layer B.Cu) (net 11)))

